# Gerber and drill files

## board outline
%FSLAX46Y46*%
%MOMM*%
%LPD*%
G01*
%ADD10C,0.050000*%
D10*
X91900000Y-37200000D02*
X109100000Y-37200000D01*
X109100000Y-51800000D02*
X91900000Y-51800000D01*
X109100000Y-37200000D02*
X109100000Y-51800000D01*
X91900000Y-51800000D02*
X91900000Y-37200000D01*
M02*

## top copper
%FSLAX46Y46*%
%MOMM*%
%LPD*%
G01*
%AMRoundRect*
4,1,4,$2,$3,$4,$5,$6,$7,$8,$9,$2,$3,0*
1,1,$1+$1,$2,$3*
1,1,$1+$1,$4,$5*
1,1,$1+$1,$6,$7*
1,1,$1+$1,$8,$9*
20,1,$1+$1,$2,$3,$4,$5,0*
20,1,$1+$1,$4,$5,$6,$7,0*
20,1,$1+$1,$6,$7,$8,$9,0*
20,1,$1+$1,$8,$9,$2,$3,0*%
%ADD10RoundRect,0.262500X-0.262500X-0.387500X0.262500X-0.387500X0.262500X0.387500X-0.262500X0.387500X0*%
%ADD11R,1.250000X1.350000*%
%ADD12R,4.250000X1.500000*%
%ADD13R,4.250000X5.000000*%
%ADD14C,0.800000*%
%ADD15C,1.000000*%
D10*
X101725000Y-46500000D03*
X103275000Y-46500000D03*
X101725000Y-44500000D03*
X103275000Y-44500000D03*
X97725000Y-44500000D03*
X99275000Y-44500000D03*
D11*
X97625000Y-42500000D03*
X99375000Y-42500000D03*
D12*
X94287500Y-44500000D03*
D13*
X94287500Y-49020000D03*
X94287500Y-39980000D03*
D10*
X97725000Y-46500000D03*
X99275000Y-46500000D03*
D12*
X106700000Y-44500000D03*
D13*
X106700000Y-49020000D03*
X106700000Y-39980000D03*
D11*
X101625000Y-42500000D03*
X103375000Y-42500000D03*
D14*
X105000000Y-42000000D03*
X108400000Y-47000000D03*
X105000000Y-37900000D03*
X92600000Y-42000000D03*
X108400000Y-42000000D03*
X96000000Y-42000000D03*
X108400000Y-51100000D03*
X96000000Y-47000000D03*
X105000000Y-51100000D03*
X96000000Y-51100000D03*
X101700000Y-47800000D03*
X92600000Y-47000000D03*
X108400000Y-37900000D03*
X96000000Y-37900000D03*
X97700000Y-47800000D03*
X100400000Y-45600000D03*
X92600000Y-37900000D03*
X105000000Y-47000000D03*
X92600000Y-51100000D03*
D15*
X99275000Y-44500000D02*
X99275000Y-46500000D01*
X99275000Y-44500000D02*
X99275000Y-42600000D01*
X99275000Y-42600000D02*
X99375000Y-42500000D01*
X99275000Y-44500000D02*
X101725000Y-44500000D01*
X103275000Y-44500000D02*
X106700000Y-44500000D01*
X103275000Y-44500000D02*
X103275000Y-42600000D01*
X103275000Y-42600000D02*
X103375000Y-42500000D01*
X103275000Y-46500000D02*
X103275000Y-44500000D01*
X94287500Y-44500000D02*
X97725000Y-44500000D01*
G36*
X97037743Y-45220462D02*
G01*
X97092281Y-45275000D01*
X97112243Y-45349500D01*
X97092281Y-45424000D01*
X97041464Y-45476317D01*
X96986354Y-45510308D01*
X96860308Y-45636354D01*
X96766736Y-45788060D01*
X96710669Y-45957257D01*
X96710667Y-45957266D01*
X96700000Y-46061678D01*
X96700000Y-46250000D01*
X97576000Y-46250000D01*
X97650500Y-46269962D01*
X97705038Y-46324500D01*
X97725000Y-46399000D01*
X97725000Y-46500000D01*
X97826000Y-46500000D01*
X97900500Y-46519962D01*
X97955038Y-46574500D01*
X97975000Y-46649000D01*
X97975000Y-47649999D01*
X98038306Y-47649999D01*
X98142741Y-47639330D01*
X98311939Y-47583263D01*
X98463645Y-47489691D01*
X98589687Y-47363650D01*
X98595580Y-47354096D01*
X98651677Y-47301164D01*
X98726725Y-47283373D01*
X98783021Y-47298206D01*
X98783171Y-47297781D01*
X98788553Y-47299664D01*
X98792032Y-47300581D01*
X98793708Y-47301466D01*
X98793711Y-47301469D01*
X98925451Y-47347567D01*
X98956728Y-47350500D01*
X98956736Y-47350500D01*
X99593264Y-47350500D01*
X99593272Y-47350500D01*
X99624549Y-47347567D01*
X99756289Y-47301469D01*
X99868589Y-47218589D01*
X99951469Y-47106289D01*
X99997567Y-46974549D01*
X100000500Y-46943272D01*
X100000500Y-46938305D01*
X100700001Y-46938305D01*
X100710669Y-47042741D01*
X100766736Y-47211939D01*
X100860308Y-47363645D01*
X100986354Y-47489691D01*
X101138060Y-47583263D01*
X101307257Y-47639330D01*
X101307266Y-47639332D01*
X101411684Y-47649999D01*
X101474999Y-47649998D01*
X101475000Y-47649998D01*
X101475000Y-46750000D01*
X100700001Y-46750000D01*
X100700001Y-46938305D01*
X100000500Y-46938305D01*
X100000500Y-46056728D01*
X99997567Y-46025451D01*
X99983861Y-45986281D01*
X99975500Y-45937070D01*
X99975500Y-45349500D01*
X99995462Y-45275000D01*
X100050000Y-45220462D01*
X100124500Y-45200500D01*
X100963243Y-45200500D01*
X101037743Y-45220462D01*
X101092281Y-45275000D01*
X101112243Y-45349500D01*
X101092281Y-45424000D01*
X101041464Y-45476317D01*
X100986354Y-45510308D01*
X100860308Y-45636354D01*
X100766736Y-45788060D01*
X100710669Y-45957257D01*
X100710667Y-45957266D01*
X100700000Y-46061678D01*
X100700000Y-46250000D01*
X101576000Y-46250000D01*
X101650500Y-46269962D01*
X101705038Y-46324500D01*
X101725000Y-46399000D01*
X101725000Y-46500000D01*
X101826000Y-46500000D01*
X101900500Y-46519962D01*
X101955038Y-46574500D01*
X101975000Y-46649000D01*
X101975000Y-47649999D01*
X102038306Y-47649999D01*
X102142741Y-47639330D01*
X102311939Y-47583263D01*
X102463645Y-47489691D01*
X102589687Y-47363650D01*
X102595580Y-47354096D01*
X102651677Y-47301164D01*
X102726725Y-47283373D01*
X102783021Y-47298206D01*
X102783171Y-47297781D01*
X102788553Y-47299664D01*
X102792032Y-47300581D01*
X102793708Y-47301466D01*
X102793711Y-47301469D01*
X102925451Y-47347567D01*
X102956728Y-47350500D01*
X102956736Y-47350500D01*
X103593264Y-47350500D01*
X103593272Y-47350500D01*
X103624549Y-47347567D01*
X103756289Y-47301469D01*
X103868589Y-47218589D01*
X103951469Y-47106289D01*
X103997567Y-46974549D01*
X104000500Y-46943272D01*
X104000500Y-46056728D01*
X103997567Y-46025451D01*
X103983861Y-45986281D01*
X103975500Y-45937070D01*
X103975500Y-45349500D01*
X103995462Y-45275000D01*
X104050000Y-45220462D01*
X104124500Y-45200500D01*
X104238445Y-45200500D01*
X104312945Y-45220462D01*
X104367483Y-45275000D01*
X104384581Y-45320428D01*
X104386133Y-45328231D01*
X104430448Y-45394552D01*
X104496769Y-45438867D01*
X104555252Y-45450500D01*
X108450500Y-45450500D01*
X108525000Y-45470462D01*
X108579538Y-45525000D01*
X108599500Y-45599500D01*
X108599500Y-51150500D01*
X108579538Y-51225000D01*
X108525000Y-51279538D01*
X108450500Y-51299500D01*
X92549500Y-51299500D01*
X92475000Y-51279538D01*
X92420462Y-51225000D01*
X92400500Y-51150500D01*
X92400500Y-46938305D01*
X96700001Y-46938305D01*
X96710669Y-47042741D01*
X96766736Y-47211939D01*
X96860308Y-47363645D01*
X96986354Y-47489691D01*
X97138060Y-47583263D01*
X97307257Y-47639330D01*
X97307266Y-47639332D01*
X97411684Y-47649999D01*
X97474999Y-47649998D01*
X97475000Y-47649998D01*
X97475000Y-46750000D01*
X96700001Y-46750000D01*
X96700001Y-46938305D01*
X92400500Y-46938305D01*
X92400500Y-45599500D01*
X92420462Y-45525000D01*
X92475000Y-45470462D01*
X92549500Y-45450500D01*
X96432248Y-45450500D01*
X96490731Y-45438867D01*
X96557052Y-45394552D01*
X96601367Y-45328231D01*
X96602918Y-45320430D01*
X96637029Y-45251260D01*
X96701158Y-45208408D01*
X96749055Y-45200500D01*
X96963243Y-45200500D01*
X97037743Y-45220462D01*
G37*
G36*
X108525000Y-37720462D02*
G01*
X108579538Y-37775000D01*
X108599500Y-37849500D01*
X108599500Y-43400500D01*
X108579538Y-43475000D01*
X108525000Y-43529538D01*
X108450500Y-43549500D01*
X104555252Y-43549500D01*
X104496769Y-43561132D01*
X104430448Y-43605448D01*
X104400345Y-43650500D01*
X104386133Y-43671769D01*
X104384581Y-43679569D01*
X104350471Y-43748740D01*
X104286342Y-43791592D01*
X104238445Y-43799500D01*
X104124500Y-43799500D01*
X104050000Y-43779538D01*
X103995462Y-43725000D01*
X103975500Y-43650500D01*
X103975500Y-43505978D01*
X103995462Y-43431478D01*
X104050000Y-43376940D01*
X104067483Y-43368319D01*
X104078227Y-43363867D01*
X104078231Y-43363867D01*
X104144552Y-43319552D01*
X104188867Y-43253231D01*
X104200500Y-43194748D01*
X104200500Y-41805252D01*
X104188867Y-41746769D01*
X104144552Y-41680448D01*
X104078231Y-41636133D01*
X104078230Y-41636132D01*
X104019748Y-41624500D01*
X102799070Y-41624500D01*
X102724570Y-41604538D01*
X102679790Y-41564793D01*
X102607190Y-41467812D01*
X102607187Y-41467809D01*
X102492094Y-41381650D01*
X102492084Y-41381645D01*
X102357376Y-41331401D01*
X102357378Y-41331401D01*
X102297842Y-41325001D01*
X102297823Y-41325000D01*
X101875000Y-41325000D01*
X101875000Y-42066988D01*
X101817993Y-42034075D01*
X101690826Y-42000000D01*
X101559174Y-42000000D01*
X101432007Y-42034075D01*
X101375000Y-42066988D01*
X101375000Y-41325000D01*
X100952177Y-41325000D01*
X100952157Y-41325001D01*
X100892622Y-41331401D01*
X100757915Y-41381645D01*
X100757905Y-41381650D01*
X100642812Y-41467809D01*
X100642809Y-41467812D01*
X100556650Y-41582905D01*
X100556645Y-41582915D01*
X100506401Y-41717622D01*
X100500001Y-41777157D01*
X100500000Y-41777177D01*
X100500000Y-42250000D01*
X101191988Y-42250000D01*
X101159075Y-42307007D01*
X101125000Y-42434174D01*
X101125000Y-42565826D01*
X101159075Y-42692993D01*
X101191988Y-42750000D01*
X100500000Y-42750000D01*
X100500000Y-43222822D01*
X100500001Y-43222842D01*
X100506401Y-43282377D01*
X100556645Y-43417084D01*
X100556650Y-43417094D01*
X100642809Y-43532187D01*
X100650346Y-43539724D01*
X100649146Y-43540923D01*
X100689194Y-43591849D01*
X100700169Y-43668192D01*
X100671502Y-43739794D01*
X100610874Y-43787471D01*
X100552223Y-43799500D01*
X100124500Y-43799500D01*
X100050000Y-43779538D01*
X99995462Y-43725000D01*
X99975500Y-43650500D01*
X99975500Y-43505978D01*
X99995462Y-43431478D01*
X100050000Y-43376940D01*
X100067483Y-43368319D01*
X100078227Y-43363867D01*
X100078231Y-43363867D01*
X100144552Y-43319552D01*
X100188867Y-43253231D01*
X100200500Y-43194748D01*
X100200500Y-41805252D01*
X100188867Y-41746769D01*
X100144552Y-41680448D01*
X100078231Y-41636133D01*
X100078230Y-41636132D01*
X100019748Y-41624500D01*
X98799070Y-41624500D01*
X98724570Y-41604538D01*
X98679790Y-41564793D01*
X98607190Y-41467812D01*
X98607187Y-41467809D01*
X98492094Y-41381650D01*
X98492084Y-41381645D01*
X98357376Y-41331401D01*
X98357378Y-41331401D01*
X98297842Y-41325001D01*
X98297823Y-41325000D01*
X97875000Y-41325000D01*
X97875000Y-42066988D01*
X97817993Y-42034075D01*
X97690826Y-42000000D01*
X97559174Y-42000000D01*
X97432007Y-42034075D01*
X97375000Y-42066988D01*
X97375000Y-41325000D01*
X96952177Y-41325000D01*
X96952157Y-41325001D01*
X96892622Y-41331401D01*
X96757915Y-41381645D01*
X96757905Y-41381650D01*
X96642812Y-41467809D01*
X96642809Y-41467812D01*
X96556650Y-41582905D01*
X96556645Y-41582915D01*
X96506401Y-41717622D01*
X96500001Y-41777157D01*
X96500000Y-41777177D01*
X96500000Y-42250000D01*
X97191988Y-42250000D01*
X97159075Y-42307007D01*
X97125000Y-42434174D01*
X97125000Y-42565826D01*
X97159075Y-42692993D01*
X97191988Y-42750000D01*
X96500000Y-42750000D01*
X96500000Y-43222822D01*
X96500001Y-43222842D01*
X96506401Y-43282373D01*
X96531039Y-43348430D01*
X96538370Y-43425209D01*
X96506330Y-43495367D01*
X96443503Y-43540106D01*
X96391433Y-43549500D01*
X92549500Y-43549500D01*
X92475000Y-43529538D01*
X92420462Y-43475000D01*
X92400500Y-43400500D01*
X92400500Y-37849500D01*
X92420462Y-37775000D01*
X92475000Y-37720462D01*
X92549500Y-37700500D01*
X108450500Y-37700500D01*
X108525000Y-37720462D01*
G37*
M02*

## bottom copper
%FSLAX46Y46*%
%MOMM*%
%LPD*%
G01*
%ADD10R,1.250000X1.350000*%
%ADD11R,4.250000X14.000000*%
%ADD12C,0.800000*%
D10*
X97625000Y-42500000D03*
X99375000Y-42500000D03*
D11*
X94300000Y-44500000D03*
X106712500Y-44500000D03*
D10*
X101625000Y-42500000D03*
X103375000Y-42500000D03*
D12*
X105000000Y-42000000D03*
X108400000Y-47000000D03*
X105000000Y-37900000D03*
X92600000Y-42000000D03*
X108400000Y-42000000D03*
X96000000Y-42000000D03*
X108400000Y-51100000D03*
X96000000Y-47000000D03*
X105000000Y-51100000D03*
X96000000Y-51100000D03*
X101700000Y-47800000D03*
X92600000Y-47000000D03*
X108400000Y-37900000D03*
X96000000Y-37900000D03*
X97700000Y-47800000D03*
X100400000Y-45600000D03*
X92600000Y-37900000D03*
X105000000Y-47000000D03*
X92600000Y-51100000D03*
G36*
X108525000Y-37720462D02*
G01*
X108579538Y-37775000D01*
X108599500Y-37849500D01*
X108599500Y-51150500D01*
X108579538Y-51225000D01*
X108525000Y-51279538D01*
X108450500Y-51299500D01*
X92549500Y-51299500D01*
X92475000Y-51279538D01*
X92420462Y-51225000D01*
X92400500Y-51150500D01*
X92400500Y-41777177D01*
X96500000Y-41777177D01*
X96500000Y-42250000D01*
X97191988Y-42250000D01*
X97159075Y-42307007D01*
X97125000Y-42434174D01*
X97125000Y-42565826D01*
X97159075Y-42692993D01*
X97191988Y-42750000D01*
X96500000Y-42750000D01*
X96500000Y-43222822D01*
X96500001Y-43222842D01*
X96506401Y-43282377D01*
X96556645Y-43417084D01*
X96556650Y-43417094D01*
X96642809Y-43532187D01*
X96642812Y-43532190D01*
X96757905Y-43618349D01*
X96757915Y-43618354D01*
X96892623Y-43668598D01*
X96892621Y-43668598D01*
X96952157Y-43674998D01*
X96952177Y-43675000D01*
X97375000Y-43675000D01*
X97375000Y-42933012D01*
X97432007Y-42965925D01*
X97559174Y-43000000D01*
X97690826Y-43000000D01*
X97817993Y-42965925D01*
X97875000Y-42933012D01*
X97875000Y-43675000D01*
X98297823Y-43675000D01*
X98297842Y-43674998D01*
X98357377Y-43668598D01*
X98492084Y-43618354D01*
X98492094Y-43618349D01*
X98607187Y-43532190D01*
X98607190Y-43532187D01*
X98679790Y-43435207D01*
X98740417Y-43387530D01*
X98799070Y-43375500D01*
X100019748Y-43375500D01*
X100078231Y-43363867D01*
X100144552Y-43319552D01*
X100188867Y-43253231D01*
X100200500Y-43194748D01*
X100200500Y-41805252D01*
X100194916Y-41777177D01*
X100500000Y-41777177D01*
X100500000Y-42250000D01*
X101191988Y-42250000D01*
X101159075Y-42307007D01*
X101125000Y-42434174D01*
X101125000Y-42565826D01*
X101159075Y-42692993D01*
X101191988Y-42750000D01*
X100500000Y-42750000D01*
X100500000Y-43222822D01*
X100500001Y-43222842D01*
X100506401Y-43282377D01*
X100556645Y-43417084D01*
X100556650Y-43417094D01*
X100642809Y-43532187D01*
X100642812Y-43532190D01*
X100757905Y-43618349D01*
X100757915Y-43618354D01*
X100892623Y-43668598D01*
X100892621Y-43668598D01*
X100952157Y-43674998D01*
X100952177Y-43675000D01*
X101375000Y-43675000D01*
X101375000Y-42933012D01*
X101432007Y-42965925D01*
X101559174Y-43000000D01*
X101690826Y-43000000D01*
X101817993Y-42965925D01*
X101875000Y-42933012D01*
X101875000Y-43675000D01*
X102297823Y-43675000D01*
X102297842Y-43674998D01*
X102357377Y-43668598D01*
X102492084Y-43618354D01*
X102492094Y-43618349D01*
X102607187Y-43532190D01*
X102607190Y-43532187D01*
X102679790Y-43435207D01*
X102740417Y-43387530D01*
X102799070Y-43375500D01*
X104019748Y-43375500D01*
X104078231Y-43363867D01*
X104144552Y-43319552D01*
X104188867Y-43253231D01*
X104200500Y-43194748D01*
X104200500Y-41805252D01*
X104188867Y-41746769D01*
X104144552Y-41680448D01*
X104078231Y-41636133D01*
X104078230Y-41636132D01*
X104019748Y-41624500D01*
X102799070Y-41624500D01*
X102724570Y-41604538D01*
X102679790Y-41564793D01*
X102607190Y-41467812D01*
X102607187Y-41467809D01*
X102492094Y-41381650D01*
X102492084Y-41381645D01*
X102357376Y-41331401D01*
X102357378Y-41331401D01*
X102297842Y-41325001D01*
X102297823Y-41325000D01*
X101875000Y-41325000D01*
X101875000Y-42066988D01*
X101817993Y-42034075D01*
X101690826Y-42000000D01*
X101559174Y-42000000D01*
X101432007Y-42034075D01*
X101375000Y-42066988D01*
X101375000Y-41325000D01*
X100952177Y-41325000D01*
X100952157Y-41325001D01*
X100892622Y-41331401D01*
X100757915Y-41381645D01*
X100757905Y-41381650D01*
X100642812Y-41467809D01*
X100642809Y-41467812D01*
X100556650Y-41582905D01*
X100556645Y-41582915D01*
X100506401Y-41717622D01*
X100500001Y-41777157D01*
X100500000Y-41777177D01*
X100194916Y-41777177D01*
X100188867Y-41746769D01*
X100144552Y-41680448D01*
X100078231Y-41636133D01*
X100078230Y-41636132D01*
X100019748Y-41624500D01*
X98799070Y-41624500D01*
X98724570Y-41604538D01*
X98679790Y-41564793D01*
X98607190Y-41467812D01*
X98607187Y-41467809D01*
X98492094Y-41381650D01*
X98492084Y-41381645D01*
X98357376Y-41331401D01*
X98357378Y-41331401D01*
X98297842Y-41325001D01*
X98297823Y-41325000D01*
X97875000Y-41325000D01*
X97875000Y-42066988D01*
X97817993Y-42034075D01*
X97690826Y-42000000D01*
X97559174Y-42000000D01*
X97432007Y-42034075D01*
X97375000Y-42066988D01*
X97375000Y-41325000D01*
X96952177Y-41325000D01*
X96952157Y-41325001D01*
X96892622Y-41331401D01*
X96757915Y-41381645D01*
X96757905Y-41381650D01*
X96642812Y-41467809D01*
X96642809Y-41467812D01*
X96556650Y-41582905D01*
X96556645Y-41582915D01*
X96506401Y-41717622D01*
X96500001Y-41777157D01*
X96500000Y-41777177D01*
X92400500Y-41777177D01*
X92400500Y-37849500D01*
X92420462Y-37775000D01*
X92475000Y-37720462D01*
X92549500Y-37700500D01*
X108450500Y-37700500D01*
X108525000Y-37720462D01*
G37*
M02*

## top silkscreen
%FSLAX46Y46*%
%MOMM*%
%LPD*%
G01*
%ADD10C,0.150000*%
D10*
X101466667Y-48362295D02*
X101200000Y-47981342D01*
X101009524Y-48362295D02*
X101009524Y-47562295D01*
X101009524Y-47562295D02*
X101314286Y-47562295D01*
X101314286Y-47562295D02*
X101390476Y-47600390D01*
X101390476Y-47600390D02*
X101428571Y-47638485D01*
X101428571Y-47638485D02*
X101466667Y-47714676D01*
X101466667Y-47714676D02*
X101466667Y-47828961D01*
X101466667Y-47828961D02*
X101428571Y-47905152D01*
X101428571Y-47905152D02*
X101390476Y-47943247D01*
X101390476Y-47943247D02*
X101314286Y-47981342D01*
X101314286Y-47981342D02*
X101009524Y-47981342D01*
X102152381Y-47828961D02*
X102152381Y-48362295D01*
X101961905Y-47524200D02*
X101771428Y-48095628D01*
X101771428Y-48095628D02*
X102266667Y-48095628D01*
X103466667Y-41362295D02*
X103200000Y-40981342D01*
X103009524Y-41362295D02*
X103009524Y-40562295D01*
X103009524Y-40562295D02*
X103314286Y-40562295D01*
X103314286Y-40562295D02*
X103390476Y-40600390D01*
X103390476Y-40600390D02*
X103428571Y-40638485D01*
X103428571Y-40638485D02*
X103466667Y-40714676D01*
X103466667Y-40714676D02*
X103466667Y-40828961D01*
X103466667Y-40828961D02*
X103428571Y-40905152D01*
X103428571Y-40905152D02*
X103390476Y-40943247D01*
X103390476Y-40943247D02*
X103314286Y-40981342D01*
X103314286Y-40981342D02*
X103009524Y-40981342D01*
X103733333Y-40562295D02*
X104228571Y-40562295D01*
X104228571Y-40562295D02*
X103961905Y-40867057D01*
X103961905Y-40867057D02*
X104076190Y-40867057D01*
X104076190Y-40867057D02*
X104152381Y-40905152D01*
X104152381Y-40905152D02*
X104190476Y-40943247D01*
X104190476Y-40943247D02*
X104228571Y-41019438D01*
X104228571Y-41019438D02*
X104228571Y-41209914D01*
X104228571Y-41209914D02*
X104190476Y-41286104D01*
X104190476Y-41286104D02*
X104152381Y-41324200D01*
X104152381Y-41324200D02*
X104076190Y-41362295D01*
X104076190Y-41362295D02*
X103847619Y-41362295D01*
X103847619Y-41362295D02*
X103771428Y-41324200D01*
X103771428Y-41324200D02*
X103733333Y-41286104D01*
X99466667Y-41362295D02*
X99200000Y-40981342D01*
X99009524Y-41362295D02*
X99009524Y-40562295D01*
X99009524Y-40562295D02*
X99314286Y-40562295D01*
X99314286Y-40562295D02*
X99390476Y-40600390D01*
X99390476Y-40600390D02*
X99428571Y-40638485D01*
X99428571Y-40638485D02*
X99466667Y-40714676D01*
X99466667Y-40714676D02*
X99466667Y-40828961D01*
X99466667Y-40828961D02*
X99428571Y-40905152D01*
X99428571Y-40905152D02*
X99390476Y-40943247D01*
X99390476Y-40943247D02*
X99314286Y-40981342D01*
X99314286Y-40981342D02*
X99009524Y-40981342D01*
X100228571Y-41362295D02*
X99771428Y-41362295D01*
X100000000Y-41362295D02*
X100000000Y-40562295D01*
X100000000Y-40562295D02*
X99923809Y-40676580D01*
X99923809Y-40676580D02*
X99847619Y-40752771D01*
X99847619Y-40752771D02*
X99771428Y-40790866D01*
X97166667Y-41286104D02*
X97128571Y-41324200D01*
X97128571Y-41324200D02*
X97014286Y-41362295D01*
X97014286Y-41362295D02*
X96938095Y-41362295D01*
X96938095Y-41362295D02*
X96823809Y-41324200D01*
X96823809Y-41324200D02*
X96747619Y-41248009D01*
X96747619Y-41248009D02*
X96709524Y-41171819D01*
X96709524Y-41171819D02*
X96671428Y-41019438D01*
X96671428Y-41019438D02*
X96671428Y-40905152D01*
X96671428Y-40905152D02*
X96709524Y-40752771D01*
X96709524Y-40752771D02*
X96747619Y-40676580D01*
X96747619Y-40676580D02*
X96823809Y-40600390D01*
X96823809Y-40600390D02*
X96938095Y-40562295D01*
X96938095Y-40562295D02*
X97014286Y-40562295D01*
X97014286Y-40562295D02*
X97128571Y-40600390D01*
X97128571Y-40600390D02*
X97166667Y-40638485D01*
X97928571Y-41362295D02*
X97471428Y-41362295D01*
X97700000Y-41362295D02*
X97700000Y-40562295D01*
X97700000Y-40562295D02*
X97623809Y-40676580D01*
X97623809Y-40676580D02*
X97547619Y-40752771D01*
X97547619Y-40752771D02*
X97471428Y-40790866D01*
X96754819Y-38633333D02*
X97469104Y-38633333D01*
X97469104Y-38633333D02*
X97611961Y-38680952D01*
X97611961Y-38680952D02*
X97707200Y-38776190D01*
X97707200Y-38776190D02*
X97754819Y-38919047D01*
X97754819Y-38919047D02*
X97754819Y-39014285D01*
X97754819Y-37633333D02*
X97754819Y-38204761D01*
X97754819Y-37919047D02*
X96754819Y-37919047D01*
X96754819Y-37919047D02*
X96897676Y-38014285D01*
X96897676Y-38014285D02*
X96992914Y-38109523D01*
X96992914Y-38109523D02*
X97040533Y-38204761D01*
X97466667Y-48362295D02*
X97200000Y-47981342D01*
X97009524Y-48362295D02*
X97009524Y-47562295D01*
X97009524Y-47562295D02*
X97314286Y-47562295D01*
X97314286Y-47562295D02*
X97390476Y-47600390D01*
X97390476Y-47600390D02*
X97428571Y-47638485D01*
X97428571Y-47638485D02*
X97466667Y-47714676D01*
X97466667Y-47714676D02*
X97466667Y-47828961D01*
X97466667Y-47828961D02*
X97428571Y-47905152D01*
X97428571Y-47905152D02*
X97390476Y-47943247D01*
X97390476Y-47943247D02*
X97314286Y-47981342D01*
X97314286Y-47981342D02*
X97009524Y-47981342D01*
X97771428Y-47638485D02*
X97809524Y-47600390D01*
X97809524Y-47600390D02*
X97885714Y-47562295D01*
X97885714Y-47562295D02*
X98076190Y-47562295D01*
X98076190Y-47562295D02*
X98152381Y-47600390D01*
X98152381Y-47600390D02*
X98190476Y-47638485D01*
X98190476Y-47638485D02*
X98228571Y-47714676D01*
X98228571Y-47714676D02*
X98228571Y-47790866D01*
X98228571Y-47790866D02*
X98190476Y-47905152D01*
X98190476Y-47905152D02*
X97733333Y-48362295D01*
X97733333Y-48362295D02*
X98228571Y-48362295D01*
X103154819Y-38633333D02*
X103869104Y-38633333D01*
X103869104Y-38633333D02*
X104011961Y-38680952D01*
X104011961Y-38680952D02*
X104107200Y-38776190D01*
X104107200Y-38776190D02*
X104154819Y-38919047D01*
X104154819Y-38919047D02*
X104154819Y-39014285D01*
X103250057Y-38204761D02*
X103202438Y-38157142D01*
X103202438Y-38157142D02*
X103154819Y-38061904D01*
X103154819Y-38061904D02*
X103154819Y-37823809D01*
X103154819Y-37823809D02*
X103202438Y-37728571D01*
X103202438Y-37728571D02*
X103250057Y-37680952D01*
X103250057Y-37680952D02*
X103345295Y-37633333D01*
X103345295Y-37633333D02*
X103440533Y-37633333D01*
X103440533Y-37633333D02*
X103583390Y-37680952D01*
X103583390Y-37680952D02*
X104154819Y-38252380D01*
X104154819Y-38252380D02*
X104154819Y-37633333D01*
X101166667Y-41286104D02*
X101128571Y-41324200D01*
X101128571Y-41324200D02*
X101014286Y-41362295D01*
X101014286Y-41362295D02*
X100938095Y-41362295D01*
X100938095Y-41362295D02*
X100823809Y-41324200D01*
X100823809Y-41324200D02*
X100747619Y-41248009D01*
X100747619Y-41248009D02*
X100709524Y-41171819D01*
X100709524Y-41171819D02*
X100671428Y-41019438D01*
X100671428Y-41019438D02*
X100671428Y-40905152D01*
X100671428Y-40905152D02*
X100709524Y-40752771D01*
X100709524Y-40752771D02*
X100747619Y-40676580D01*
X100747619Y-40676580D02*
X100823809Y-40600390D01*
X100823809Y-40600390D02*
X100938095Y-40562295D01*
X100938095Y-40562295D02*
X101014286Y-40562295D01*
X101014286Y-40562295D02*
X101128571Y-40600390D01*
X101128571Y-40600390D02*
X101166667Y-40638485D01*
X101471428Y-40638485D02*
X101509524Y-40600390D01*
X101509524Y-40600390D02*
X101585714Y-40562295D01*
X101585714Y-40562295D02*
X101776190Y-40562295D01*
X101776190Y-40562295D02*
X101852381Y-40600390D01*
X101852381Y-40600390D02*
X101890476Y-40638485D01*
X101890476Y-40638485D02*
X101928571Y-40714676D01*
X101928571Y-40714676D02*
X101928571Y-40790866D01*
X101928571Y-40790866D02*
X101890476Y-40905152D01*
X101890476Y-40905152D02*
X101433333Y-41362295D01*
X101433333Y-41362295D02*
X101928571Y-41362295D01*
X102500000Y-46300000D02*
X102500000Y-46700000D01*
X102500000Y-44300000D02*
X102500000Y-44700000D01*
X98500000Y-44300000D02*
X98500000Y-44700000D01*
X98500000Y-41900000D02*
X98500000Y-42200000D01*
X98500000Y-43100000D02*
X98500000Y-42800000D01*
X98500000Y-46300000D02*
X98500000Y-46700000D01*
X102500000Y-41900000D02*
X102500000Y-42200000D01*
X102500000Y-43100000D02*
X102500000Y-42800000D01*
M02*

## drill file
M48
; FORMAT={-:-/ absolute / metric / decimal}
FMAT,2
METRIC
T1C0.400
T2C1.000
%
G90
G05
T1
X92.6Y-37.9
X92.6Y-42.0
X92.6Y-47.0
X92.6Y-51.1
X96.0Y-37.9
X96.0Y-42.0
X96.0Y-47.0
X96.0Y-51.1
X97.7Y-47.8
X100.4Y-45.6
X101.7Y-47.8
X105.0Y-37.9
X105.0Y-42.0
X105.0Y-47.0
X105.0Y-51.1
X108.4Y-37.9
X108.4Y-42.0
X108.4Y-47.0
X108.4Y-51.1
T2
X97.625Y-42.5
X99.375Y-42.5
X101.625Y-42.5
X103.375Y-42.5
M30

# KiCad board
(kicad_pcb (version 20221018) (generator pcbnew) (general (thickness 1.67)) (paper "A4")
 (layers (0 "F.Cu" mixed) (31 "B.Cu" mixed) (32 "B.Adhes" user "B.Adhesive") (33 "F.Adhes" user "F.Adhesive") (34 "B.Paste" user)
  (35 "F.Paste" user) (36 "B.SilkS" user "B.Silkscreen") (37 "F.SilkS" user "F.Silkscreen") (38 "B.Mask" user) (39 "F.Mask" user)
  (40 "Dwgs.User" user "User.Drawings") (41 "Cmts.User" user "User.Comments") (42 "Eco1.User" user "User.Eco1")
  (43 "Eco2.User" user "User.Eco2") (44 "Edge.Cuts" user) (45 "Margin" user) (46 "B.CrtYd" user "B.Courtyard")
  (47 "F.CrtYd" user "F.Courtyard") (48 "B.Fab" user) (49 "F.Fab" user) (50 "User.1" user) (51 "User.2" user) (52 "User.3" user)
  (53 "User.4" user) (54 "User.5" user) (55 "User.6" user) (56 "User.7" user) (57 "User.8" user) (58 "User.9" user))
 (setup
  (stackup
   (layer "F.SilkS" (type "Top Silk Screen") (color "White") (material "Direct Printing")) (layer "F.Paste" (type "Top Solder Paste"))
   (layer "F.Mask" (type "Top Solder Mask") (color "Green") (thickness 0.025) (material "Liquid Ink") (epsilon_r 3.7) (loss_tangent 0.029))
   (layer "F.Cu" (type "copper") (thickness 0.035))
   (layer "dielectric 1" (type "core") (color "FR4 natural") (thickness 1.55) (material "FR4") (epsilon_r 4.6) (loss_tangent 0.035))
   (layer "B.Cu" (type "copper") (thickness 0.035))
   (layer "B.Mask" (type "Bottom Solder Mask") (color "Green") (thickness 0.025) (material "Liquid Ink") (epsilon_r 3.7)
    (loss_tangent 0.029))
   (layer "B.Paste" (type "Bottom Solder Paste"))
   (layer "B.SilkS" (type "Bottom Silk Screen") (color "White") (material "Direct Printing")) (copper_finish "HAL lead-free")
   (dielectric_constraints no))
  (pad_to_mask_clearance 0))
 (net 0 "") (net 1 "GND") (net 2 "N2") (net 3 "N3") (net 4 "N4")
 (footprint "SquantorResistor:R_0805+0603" (layer "F.Cu") (at 102.5 46.5)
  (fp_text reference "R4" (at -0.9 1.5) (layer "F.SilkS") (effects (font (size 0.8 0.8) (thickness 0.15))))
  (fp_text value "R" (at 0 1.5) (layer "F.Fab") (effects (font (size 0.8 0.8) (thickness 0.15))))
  (fp_line (start 0 -0.2) (end 0 0.2) (stroke (width 0.15) (type solid)) (layer "F.SilkS"))
  (pad "1" smd roundrect (at -0.775 0) (size 1.05 1.3) (layers "F.Cu" "F.Paste" "F.Mask") (roundrect_rratio 0.25) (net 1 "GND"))
  (pad "2" smd roundrect (at 0.775 0) (size 1.05 1.3) (layers "F.Cu" "F.Paste" "F.Mask") (roundrect_rratio 0.25) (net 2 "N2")))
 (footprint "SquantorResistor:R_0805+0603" (layer "F.Cu") (at 102.5 44.5)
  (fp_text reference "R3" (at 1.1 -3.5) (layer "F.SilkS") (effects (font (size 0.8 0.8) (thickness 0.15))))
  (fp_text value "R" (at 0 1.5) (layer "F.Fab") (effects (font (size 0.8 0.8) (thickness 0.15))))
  (fp_line (start 0 -0.2) (end 0 0.2) (stroke (width 0.15) (type solid)) (layer "F.SilkS"))
  (pad "1" smd roundrect (at -0.775 0) (size 1.05 1.3) (layers "F.Cu" "F.Paste" "F.Mask") (roundrect_rratio 0.25) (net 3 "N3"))
  (pad "2" smd roundrect (at 0.775 0) (size 1.05 1.3) (layers "F.Cu" "F.Paste" "F.Mask") (roundrect_rratio 0.25) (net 2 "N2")))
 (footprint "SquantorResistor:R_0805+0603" (layer "F.Cu") (at 98.5 44.5)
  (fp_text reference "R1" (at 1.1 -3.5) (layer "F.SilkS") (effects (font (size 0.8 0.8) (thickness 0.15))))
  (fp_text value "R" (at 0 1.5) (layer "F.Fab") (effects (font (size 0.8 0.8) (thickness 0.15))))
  (fp_line (start 0 -0.2) (end 0 0.2) (stroke (width 0.15) (type solid)) (layer "F.SilkS"))
  (pad "1" smd roundrect (at -0.775 0) (size 1.05 1.3) (layers "F.Cu" "F.Paste" "F.Mask") (roundrect_rratio 0.25) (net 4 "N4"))
  (pad "2" smd roundrect (at 0.775 0) (size 1.05 1.3) (layers "F.Cu" "F.Paste" "F.Mask") (roundrect_rratio 0.25) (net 3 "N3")))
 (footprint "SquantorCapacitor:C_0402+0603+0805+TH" (layer "F.Cu") (at 98.5 42.5)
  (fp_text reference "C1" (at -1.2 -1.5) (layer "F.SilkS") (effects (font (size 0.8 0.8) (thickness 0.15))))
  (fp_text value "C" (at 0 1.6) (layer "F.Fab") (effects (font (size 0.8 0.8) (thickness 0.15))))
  (fp_line (start 0 -0.6) (end 0 -0.3) (stroke (width 0.15) (type default)) (layer "F.SilkS"))
  (fp_line (start 0 0.6) (end 0 0.3) (stroke (width 0.15) (type default)) (layer "F.SilkS"))
  (pad "1" thru_hole rect (at -0.875 0) (size 1.25 1.35) (drill 1) (layers "*.Cu" "*.Mask") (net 1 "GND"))
  (pad "2" thru_hole rect (at 0.875 0) (size 1.25 1.35) (drill 1) (layers "*.Cu" "*.Mask") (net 3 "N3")))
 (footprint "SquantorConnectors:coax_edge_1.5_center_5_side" (layer "F.Cu") (at 94.2875 44.5 90)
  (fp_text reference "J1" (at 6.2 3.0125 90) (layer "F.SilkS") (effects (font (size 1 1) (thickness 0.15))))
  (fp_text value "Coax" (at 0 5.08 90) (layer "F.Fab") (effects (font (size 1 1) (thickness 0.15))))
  (pad "1" smd rect (at 0 0 90) (size 1.5 4.25) (layers "F.Cu" "F.Paste" "F.Mask") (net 4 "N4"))
  (pad "2" smd rect (at -4.52 0 90) (size 5 4.25) (layers "F.Cu" "F.Paste" "F.Mask") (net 1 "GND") (zone_connect 2))
  (pad "2" smd rect (at 0 0.0125 90) (size 14 4.25) (layers "B.Cu" "B.Paste" "B.Mask") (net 1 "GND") (zone_connect 2))
  (pad "2" smd rect (at 4.52 0 90) (size 5 4.25) (layers "F.Cu" "F.Paste" "F.Mask") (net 1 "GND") (zone_connect 2)))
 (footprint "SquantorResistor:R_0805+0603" (layer "F.Cu") (at 98.5 46.5)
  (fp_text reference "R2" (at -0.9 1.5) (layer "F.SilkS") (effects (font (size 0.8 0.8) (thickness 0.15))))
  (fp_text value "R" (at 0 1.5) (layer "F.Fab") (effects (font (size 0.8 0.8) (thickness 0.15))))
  (fp_line (start 0 -0.2) (end 0 0.2) (stroke (width 0.15) (type solid)) (layer "F.SilkS"))
  (pad "1" smd roundrect (at -0.775 0) (size 1.05 1.3) (layers "F.Cu" "F.Paste" "F.Mask") (roundrect_rratio 0.25) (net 1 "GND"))
  (pad "2" smd roundrect (at 0.775 0) (size 1.05 1.3) (layers "F.Cu" "F.Paste" "F.Mask") (roundrect_rratio 0.25) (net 3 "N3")))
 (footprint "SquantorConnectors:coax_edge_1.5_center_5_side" (layer "F.Cu") (at 106.7 44.5 90)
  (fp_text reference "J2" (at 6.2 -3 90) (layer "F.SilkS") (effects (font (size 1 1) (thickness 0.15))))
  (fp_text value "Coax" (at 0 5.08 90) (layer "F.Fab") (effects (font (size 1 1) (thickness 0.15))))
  (pad "1" smd rect (at 0 0 90) (size 1.5 4.25) (layers "F.Cu" "F.Paste" "F.Mask") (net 2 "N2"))
  (pad "2" smd rect (at -4.52 0 90) (size 5 4.25) (layers "F.Cu" "F.Paste" "F.Mask") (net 1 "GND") (zone_connect 2))
  (pad "2" smd rect (at 0 0.0125 90) (size 14 4.25) (layers "B.Cu" "B.Paste" "B.Mask") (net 1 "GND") (zone_connect 2))
  (pad "2" smd rect (at 4.52 0 90) (size 5 4.25) (layers "F.Cu" "F.Paste" "F.Mask") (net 1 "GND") (zone_connect 2)))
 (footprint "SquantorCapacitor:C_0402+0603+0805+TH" (layer "F.Cu") (at 102.5 42.5)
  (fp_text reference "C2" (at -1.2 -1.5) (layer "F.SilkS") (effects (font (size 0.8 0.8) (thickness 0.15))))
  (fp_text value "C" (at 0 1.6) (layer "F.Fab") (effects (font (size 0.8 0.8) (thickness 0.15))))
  (fp_line (start 0 -0.6) (end 0 -0.3) (stroke (width 0.15) (type default)) (layer "F.SilkS"))
  (fp_line (start 0 0.6) (end 0 0.3) (stroke (width 0.15) (type default)) (layer "F.SilkS"))
  (pad "1" thru_hole rect (at -0.875 0) (size 1.25 1.35) (drill 1) (layers "*.Cu" "*.Mask") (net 1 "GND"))
  (pad "2" thru_hole rect (at 0.875 0) (size 1.25 1.35) (drill 1) (layers "*.Cu" "*.Mask") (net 2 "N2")))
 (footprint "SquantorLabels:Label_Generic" (layer "B.Cu") (at 100.5 50.7 180)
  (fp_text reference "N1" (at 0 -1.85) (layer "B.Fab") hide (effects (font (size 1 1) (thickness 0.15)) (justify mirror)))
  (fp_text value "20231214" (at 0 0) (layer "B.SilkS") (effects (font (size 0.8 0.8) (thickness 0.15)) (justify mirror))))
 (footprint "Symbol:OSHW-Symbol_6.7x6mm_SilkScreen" (layer "B.Cu") (at 100.5 47 180)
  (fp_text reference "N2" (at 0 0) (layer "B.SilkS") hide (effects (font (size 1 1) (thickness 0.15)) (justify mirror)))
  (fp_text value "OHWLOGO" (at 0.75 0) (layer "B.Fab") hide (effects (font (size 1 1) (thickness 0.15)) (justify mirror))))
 (gr_line (start 91.9 37.2) (end 109.1 37.2) (stroke (width 0.05) (type default)) (layer "Edge.Cuts"))
 (gr_line (start 109.1 51.8) (end 91.9 51.8) (stroke (width 0.05) (type default)) (layer "Edge.Cuts"))
 (gr_line (start 109.1 37.2) (end 109.1 51.8) (stroke (width 0.05) (type default)) (layer "Edge.Cuts"))
 (gr_line (start 91.9 51.8) (end 91.9 37.2) (stroke (width 0.05) (type default)) (layer "Edge.Cuts"))
 (via (at 105 42) (size 0.8) (drill 0.4) (layers "F.Cu" "B.Cu") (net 1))
 (via (at 108.4 47) (size 0.8) (drill 0.4) (layers "F.Cu" "B.Cu") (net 1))
 (via (at 105 37.9) (size 0.8) (drill 0.4) (layers "F.Cu" "B.Cu") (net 1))
 (via (at 92.6 42) (size 0.8) (drill 0.4) (layers "F.Cu" "B.Cu") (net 1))
 (via (at 108.4 42) (size 0.8) (drill 0.4) (layers "F.Cu" "B.Cu") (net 1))
 (via (at 96 42) (size 0.8) (drill 0.4) (layers "F.Cu" "B.Cu") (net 1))
 (via (at 108.4 51.1) (size 0.8) (drill 0.4) (layers "F.Cu" "B.Cu") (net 1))
 (via (at 96 47) (size 0.8) (drill 0.4) (layers "F.Cu" "B.Cu") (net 1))
 (via (at 105 51.1) (size 0.8) (drill 0.4) (layers "F.Cu" "B.Cu") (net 1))
 (via (at 96 51.1) (size 0.8) (drill 0.4) (layers "F.Cu" "B.Cu") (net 1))
 (via (at 101.7 47.8) (size 0.8) (drill 0.4) (layers "F.Cu" "B.Cu") (free) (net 1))
 (via (at 92.6 47) (size 0.8) (drill 0.4) (layers "F.Cu" "B.Cu") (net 1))
 (via (at 108.4 37.9) (size 0.8) (drill 0.4) (layers "F.Cu" "B.Cu") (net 1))
 (via (at 96 37.9) (size 0.8) (drill 0.4) (layers "F.Cu" "B.Cu") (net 1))
 (via (at 97.7 47.8) (size 0.8) (drill 0.4) (layers "F.Cu" "B.Cu") (free) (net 1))
 (via (at 100.4 45.6) (size 0.8) (drill 0.4) (layers "F.Cu" "B.Cu") (free) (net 1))
 (via (at 92.6 37.9) (size 0.8) (drill 0.4) (layers "F.Cu" "B.Cu") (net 1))
 (via (at 105 47) (size 0.8) (drill 0.4) (layers "F.Cu" "B.Cu") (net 1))
 (via (at 92.6 51.1) (size 0.8) (drill 0.4) (layers "F.Cu" "B.Cu") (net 1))
 (segment (start 99.275 44.5) (end 99.275 46.5) (width 1) (layer "F.Cu") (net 3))
 (segment (start 99.275 44.5) (end 99.275 42.6) (width 1) (layer "F.Cu") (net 3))
 (segment (start 99.275 42.6) (end 99.375 42.5) (width 1) (layer "F.Cu") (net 3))
 (segment (start 99.275 44.5) (end 101.725 44.5) (width 1) (layer "F.Cu") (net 3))
 (segment (start 103.275 44.5) (end 106.7 44.5) (width 1) (layer "F.Cu") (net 2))
 (segment (start 103.275 44.5) (end 103.275 42.6) (width 1) (layer "F.Cu") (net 2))
 (segment (start 103.275 42.6) (end 103.375 42.5) (width 1) (layer "F.Cu") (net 2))
 (segment (start 103.275 46.5) (end 103.275 44.5) (width 1) (layer "F.Cu") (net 2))
 (segment (start 94.2875 44.5) (end 97.725 44.5) (width 1) (layer "F.Cu") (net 4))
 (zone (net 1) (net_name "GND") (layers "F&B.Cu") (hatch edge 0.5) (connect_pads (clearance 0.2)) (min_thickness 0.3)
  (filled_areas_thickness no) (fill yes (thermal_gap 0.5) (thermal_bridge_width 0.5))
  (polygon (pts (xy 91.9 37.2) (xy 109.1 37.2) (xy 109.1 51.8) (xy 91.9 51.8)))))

